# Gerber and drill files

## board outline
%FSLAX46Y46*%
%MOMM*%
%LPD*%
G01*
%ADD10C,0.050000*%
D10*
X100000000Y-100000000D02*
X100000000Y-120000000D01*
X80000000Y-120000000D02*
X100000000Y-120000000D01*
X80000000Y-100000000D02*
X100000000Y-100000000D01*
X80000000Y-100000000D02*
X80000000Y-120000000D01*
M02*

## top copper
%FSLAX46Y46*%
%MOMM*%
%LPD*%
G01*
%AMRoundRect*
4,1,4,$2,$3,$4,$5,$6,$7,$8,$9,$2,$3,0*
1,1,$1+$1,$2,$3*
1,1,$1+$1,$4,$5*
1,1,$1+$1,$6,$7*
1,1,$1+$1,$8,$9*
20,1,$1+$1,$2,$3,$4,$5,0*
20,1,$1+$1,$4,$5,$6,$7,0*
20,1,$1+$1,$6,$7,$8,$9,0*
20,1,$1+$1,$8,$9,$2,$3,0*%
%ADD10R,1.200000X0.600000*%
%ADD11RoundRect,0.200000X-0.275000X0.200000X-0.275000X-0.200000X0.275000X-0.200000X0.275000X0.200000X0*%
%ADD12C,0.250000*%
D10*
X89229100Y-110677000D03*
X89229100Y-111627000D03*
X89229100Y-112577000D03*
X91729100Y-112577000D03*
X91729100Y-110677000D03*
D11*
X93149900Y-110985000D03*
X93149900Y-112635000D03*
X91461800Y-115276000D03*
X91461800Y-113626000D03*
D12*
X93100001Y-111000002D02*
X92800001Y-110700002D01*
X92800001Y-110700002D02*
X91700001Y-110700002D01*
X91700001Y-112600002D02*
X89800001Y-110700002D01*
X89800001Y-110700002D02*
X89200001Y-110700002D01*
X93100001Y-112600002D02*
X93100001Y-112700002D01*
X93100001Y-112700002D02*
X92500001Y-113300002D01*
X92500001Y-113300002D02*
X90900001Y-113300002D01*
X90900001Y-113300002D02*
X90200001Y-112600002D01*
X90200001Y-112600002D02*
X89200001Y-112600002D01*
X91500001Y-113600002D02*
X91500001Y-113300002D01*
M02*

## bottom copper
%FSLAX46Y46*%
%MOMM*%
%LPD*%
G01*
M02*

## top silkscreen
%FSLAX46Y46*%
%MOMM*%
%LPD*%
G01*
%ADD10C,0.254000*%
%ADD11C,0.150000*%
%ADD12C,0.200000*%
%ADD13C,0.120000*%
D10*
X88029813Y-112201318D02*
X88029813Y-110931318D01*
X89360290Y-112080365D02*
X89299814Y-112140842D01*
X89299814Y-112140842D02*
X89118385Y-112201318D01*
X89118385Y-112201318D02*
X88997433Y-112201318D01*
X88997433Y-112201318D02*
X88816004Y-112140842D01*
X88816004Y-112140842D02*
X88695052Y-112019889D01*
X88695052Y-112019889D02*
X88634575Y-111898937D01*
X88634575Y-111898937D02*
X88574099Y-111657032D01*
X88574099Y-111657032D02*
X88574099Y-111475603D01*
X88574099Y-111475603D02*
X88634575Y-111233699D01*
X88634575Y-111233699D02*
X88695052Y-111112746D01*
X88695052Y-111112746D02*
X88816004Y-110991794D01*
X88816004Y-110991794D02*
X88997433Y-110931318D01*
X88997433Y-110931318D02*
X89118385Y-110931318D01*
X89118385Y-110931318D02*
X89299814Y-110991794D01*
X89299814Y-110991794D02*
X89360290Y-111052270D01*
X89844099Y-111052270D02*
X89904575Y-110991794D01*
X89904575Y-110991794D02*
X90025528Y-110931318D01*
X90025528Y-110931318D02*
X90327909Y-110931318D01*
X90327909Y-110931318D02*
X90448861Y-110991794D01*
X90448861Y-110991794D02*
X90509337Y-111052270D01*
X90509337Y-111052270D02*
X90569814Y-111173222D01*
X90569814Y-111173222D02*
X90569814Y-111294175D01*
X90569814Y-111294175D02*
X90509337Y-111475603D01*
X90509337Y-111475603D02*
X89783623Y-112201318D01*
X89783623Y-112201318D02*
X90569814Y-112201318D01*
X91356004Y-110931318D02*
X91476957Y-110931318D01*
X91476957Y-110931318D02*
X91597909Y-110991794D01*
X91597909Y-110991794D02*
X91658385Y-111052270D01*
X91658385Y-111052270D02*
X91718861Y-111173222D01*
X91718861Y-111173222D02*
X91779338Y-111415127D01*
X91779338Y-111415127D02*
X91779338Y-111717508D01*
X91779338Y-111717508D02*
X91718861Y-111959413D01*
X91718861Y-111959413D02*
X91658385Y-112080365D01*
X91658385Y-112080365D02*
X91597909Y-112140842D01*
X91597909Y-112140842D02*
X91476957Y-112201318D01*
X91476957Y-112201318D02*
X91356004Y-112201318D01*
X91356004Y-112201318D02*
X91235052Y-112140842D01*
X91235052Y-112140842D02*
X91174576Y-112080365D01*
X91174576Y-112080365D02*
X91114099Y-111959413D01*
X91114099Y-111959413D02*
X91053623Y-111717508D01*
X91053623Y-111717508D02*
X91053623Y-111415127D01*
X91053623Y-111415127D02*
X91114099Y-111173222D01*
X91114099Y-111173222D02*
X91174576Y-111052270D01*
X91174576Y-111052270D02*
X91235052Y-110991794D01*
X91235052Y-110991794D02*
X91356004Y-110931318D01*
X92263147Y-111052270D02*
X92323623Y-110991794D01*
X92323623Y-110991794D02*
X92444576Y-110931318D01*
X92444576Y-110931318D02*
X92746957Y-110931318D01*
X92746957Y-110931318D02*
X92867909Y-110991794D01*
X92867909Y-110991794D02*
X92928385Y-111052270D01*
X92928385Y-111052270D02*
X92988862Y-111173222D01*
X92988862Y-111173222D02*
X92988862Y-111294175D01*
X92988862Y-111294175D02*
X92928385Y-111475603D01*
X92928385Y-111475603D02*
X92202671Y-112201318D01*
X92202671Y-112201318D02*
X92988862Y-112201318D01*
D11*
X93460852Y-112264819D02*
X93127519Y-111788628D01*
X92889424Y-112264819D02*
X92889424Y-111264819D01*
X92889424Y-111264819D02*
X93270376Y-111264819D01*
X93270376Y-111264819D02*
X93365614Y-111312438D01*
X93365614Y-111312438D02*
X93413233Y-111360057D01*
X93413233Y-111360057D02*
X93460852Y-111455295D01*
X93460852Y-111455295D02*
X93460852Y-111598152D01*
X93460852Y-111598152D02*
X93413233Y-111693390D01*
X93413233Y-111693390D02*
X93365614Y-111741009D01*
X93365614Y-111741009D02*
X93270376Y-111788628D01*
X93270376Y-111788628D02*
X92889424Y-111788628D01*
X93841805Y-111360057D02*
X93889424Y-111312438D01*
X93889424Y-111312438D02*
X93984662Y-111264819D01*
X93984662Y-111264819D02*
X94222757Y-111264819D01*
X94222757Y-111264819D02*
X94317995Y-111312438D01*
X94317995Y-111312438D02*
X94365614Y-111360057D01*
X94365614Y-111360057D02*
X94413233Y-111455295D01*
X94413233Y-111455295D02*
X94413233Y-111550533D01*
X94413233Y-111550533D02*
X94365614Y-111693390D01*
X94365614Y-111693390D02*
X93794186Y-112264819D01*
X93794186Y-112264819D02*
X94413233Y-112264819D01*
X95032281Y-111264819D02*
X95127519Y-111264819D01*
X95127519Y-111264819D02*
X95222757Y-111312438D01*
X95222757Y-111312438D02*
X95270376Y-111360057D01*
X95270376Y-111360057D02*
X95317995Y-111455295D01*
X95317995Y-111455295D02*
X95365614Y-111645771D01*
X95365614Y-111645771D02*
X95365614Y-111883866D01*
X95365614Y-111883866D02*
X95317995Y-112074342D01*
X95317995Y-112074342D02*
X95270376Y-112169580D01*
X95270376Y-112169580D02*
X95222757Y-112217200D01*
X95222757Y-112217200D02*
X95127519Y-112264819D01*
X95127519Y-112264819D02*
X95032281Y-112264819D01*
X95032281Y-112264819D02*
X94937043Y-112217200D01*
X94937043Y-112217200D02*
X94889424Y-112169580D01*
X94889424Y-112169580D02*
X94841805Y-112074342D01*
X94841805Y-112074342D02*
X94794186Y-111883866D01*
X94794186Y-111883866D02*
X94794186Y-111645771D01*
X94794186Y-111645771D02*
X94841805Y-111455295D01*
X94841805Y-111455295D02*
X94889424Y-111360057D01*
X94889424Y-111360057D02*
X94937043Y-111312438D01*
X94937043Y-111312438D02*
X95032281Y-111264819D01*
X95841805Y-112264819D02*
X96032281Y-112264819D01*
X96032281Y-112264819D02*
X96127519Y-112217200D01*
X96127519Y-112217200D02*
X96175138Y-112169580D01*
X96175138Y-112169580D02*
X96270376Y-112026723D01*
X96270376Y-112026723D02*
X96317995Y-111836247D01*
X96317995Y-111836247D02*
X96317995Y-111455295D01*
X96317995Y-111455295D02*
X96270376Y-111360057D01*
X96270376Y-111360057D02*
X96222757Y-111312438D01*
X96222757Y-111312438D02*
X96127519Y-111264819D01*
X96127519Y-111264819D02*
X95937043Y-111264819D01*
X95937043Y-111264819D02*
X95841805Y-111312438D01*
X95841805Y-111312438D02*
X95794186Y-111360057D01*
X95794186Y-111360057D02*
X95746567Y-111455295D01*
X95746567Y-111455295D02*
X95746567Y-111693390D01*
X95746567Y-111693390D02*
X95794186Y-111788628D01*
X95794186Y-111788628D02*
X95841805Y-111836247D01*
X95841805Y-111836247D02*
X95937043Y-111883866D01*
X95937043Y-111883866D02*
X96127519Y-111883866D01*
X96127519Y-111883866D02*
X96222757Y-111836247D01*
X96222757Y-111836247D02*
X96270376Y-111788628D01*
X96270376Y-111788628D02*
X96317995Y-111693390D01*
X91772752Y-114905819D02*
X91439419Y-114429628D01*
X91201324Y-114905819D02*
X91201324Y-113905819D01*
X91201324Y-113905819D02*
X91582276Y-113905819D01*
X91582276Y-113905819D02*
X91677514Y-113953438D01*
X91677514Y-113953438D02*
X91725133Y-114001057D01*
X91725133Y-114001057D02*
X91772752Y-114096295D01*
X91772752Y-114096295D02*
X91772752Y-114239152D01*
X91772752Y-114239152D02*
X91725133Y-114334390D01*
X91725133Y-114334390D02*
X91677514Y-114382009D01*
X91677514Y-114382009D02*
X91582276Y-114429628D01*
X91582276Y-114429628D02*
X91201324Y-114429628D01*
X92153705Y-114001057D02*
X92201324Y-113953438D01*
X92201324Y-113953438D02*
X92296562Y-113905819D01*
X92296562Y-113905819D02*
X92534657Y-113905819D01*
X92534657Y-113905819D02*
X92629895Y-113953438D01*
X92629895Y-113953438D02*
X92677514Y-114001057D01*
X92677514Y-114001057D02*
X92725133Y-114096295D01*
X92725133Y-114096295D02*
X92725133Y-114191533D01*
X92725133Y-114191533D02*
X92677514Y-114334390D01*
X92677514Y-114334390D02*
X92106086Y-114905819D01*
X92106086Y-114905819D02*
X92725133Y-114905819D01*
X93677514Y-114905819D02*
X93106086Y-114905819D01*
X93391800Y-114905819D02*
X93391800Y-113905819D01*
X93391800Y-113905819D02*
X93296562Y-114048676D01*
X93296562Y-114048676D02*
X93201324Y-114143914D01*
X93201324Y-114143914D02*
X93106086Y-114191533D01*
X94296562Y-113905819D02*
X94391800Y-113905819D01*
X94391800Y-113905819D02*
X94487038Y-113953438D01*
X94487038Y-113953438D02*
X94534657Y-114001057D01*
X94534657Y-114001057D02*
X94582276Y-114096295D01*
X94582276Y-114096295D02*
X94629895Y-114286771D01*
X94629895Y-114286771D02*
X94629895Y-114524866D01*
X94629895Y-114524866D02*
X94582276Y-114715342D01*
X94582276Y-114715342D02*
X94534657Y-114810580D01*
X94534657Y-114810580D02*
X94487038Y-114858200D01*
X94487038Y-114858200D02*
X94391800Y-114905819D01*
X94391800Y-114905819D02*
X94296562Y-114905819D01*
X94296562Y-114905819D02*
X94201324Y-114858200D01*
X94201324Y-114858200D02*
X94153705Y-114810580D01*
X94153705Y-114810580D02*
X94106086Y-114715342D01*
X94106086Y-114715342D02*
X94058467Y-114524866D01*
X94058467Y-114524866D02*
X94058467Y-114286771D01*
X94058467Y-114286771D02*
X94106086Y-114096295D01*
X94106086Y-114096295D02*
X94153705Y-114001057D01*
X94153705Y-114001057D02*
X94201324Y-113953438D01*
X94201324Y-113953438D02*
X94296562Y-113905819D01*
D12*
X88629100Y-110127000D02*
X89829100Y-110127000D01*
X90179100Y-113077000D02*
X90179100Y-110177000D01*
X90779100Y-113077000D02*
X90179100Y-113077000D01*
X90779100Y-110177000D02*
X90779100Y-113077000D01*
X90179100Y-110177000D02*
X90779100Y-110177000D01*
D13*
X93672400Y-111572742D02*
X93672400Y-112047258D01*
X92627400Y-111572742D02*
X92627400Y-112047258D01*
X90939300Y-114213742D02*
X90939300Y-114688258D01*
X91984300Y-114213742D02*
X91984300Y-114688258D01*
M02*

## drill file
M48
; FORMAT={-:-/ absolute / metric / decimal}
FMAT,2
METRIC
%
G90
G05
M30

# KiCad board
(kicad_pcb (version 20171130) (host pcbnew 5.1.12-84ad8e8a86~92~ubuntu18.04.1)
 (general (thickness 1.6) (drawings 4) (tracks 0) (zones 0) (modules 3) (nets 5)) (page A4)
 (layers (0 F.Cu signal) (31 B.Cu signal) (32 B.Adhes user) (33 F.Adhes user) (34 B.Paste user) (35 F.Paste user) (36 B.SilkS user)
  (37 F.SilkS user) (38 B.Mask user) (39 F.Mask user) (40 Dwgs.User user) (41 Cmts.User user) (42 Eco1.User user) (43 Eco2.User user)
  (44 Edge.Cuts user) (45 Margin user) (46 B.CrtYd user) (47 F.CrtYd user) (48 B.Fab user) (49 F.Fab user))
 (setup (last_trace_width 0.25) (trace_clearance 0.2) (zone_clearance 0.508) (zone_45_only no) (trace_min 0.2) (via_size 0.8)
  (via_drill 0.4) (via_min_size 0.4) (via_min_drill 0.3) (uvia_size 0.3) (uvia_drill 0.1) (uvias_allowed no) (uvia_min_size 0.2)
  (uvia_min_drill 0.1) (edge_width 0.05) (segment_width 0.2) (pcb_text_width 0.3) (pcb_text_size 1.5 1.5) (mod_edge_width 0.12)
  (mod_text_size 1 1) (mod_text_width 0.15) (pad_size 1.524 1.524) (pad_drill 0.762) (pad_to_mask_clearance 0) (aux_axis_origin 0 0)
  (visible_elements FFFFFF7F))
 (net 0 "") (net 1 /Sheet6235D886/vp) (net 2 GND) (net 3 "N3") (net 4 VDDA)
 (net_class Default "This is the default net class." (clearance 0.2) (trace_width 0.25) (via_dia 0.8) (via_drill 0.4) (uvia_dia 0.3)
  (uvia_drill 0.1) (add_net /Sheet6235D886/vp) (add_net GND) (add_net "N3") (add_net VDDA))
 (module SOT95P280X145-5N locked (layer F.Cu) (at 90.479100 111.627000)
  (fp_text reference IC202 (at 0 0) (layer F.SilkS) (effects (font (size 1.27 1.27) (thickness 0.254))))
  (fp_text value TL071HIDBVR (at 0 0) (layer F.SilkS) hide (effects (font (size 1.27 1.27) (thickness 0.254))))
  (fp_line (start -1.85 -1.5) (end -0.65 -1.5) (layer F.SilkS) (width 0.2))
  (fp_line (start -0.3 1.45) (end -0.3 -1.45) (layer F.SilkS) (width 0.2))
  (fp_line (start 0.3 1.45) (end -0.3 1.45) (layer F.SilkS) (width 0.2))
  (fp_line (start 0.3 -1.45) (end 0.3 1.45) (layer F.SilkS) (width 0.2))
  (fp_line (start -0.3 -1.45) (end 0.3 -1.45) (layer F.SilkS) (width 0.2))
  (pad 1 smd rect (at -1.25 -0.95 90.000000) (size 0.6 1.2) (layers F.Cu F.Mask F.Paste) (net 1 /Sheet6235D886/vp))
  (pad 2 smd rect (at -1.25 0 90.000000) (size 0.6 1.2) (layers F.Cu F.Mask F.Paste) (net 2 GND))
  (pad 3 smd rect (at -1.25 0.95 90.000000) (size 0.6 1.2) (layers F.Cu F.Mask F.Paste) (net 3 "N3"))
  (pad 4 smd rect (at 1.25 0.95 90.000000) (size 0.6 1.2) (layers F.Cu F.Mask F.Paste) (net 1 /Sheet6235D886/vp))
  (pad 5 smd rect (at 1.25 -0.95 90.000000) (size 0.6 1.2) (layers F.Cu F.Mask F.Paste) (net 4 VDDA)))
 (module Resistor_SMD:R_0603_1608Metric (layer F.Cu) (at 93.149900 111.810000 270.000000)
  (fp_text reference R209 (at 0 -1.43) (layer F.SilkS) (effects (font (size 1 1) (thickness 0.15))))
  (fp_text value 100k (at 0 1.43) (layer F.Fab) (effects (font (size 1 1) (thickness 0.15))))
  (fp_line (start -0.237258 -0.5225) (end 0.237258 -0.5225) (layer F.SilkS) (width 0.12))
  (fp_line (start -0.237258 0.5225) (end 0.237258 0.5225) (layer F.SilkS) (width 0.12))
  (pad 1 smd roundrect (at -0.825 0 270.000000) (size 0.8 0.95) (layers F.Cu F.Mask F.Paste) (roundrect_rratio 0.25) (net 4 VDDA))
  (pad 2 smd roundrect (at 0.825 0 270.000000) (size 0.8 0.95) (layers F.Cu F.Mask F.Paste) (roundrect_rratio 0.25) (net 3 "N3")))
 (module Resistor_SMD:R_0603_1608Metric (layer F.Cu) (at 91.461800 114.451000 270.000000)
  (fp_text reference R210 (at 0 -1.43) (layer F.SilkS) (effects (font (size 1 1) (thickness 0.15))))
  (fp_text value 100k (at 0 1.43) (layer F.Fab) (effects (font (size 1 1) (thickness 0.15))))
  (fp_line (start -0.237258 0.5225) (end 0.237258 0.5225) (layer F.SilkS) (width 0.12))
  (fp_line (start -0.237258 -0.5225) (end 0.237258 -0.5225) (layer F.SilkS) (width 0.12))
  (pad 2 smd roundrect (at 0.825 0 270.000000) (size 0.8 0.95) (layers F.Cu F.Mask F.Paste) (roundrect_rratio 0.25) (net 2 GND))
  (pad 1 smd roundrect (at -0.825 0 270.000000) (size 0.8 0.95) (layers F.Cu F.Mask F.Paste) (roundrect_rratio 0.25) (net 3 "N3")))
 (gr_line (start 100 100) (end 100 120) (layer Edge.Cuts) (width 0.05))
 (gr_line (start 80 120) (end 100 120) (layer Edge.Cuts) (width 0.05))
 (gr_line (start 80 100) (end 100 100) (layer Edge.Cuts) (width 0.05))
 (gr_line (start 80 100) (end 80 120) (layer Edge.Cuts) (width 0.05))
 (segment (start 93.100001 111.000002) (end 92.800001 110.700002) (width 0.250000) (layer F.Cu) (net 4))
 (segment (start 92.800001 110.700002) (end 91.700001 110.700002) (width 0.250000) (layer F.Cu) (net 4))
 (segment (start 91.700001 112.600002) (end 89.800001 110.700002) (width 0.250000) (layer F.Cu) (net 1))
 (segment (start 89.800001 110.700002) (end 89.200001 110.700002) (width 0.250000) (layer F.Cu) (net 1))
 (segment (start 93.100001 112.600002) (end 93.100001 112.700002) (width 0.250000) (layer F.Cu) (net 3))
 (segment (start 93.100001 112.700002) (end 92.500001 113.300002) (width 0.250000) (layer F.Cu) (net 3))
 (segment (start 92.500001 113.300002) (end 90.900001 113.300002) (width 0.250000) (layer F.Cu) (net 3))
 (segment (start 90.900001 113.300002) (end 90.200001 112.600002) (width 0.250000) (layer F.Cu) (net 3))
 (segment (start 90.200001 112.600002) (end 89.200001 112.600002) (width 0.250000) (layer F.Cu) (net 3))
 (segment (start 91.500001 113.600002) (end 91.500001 113.300002) (width 0.250000) (layer F.Cu) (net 3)))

